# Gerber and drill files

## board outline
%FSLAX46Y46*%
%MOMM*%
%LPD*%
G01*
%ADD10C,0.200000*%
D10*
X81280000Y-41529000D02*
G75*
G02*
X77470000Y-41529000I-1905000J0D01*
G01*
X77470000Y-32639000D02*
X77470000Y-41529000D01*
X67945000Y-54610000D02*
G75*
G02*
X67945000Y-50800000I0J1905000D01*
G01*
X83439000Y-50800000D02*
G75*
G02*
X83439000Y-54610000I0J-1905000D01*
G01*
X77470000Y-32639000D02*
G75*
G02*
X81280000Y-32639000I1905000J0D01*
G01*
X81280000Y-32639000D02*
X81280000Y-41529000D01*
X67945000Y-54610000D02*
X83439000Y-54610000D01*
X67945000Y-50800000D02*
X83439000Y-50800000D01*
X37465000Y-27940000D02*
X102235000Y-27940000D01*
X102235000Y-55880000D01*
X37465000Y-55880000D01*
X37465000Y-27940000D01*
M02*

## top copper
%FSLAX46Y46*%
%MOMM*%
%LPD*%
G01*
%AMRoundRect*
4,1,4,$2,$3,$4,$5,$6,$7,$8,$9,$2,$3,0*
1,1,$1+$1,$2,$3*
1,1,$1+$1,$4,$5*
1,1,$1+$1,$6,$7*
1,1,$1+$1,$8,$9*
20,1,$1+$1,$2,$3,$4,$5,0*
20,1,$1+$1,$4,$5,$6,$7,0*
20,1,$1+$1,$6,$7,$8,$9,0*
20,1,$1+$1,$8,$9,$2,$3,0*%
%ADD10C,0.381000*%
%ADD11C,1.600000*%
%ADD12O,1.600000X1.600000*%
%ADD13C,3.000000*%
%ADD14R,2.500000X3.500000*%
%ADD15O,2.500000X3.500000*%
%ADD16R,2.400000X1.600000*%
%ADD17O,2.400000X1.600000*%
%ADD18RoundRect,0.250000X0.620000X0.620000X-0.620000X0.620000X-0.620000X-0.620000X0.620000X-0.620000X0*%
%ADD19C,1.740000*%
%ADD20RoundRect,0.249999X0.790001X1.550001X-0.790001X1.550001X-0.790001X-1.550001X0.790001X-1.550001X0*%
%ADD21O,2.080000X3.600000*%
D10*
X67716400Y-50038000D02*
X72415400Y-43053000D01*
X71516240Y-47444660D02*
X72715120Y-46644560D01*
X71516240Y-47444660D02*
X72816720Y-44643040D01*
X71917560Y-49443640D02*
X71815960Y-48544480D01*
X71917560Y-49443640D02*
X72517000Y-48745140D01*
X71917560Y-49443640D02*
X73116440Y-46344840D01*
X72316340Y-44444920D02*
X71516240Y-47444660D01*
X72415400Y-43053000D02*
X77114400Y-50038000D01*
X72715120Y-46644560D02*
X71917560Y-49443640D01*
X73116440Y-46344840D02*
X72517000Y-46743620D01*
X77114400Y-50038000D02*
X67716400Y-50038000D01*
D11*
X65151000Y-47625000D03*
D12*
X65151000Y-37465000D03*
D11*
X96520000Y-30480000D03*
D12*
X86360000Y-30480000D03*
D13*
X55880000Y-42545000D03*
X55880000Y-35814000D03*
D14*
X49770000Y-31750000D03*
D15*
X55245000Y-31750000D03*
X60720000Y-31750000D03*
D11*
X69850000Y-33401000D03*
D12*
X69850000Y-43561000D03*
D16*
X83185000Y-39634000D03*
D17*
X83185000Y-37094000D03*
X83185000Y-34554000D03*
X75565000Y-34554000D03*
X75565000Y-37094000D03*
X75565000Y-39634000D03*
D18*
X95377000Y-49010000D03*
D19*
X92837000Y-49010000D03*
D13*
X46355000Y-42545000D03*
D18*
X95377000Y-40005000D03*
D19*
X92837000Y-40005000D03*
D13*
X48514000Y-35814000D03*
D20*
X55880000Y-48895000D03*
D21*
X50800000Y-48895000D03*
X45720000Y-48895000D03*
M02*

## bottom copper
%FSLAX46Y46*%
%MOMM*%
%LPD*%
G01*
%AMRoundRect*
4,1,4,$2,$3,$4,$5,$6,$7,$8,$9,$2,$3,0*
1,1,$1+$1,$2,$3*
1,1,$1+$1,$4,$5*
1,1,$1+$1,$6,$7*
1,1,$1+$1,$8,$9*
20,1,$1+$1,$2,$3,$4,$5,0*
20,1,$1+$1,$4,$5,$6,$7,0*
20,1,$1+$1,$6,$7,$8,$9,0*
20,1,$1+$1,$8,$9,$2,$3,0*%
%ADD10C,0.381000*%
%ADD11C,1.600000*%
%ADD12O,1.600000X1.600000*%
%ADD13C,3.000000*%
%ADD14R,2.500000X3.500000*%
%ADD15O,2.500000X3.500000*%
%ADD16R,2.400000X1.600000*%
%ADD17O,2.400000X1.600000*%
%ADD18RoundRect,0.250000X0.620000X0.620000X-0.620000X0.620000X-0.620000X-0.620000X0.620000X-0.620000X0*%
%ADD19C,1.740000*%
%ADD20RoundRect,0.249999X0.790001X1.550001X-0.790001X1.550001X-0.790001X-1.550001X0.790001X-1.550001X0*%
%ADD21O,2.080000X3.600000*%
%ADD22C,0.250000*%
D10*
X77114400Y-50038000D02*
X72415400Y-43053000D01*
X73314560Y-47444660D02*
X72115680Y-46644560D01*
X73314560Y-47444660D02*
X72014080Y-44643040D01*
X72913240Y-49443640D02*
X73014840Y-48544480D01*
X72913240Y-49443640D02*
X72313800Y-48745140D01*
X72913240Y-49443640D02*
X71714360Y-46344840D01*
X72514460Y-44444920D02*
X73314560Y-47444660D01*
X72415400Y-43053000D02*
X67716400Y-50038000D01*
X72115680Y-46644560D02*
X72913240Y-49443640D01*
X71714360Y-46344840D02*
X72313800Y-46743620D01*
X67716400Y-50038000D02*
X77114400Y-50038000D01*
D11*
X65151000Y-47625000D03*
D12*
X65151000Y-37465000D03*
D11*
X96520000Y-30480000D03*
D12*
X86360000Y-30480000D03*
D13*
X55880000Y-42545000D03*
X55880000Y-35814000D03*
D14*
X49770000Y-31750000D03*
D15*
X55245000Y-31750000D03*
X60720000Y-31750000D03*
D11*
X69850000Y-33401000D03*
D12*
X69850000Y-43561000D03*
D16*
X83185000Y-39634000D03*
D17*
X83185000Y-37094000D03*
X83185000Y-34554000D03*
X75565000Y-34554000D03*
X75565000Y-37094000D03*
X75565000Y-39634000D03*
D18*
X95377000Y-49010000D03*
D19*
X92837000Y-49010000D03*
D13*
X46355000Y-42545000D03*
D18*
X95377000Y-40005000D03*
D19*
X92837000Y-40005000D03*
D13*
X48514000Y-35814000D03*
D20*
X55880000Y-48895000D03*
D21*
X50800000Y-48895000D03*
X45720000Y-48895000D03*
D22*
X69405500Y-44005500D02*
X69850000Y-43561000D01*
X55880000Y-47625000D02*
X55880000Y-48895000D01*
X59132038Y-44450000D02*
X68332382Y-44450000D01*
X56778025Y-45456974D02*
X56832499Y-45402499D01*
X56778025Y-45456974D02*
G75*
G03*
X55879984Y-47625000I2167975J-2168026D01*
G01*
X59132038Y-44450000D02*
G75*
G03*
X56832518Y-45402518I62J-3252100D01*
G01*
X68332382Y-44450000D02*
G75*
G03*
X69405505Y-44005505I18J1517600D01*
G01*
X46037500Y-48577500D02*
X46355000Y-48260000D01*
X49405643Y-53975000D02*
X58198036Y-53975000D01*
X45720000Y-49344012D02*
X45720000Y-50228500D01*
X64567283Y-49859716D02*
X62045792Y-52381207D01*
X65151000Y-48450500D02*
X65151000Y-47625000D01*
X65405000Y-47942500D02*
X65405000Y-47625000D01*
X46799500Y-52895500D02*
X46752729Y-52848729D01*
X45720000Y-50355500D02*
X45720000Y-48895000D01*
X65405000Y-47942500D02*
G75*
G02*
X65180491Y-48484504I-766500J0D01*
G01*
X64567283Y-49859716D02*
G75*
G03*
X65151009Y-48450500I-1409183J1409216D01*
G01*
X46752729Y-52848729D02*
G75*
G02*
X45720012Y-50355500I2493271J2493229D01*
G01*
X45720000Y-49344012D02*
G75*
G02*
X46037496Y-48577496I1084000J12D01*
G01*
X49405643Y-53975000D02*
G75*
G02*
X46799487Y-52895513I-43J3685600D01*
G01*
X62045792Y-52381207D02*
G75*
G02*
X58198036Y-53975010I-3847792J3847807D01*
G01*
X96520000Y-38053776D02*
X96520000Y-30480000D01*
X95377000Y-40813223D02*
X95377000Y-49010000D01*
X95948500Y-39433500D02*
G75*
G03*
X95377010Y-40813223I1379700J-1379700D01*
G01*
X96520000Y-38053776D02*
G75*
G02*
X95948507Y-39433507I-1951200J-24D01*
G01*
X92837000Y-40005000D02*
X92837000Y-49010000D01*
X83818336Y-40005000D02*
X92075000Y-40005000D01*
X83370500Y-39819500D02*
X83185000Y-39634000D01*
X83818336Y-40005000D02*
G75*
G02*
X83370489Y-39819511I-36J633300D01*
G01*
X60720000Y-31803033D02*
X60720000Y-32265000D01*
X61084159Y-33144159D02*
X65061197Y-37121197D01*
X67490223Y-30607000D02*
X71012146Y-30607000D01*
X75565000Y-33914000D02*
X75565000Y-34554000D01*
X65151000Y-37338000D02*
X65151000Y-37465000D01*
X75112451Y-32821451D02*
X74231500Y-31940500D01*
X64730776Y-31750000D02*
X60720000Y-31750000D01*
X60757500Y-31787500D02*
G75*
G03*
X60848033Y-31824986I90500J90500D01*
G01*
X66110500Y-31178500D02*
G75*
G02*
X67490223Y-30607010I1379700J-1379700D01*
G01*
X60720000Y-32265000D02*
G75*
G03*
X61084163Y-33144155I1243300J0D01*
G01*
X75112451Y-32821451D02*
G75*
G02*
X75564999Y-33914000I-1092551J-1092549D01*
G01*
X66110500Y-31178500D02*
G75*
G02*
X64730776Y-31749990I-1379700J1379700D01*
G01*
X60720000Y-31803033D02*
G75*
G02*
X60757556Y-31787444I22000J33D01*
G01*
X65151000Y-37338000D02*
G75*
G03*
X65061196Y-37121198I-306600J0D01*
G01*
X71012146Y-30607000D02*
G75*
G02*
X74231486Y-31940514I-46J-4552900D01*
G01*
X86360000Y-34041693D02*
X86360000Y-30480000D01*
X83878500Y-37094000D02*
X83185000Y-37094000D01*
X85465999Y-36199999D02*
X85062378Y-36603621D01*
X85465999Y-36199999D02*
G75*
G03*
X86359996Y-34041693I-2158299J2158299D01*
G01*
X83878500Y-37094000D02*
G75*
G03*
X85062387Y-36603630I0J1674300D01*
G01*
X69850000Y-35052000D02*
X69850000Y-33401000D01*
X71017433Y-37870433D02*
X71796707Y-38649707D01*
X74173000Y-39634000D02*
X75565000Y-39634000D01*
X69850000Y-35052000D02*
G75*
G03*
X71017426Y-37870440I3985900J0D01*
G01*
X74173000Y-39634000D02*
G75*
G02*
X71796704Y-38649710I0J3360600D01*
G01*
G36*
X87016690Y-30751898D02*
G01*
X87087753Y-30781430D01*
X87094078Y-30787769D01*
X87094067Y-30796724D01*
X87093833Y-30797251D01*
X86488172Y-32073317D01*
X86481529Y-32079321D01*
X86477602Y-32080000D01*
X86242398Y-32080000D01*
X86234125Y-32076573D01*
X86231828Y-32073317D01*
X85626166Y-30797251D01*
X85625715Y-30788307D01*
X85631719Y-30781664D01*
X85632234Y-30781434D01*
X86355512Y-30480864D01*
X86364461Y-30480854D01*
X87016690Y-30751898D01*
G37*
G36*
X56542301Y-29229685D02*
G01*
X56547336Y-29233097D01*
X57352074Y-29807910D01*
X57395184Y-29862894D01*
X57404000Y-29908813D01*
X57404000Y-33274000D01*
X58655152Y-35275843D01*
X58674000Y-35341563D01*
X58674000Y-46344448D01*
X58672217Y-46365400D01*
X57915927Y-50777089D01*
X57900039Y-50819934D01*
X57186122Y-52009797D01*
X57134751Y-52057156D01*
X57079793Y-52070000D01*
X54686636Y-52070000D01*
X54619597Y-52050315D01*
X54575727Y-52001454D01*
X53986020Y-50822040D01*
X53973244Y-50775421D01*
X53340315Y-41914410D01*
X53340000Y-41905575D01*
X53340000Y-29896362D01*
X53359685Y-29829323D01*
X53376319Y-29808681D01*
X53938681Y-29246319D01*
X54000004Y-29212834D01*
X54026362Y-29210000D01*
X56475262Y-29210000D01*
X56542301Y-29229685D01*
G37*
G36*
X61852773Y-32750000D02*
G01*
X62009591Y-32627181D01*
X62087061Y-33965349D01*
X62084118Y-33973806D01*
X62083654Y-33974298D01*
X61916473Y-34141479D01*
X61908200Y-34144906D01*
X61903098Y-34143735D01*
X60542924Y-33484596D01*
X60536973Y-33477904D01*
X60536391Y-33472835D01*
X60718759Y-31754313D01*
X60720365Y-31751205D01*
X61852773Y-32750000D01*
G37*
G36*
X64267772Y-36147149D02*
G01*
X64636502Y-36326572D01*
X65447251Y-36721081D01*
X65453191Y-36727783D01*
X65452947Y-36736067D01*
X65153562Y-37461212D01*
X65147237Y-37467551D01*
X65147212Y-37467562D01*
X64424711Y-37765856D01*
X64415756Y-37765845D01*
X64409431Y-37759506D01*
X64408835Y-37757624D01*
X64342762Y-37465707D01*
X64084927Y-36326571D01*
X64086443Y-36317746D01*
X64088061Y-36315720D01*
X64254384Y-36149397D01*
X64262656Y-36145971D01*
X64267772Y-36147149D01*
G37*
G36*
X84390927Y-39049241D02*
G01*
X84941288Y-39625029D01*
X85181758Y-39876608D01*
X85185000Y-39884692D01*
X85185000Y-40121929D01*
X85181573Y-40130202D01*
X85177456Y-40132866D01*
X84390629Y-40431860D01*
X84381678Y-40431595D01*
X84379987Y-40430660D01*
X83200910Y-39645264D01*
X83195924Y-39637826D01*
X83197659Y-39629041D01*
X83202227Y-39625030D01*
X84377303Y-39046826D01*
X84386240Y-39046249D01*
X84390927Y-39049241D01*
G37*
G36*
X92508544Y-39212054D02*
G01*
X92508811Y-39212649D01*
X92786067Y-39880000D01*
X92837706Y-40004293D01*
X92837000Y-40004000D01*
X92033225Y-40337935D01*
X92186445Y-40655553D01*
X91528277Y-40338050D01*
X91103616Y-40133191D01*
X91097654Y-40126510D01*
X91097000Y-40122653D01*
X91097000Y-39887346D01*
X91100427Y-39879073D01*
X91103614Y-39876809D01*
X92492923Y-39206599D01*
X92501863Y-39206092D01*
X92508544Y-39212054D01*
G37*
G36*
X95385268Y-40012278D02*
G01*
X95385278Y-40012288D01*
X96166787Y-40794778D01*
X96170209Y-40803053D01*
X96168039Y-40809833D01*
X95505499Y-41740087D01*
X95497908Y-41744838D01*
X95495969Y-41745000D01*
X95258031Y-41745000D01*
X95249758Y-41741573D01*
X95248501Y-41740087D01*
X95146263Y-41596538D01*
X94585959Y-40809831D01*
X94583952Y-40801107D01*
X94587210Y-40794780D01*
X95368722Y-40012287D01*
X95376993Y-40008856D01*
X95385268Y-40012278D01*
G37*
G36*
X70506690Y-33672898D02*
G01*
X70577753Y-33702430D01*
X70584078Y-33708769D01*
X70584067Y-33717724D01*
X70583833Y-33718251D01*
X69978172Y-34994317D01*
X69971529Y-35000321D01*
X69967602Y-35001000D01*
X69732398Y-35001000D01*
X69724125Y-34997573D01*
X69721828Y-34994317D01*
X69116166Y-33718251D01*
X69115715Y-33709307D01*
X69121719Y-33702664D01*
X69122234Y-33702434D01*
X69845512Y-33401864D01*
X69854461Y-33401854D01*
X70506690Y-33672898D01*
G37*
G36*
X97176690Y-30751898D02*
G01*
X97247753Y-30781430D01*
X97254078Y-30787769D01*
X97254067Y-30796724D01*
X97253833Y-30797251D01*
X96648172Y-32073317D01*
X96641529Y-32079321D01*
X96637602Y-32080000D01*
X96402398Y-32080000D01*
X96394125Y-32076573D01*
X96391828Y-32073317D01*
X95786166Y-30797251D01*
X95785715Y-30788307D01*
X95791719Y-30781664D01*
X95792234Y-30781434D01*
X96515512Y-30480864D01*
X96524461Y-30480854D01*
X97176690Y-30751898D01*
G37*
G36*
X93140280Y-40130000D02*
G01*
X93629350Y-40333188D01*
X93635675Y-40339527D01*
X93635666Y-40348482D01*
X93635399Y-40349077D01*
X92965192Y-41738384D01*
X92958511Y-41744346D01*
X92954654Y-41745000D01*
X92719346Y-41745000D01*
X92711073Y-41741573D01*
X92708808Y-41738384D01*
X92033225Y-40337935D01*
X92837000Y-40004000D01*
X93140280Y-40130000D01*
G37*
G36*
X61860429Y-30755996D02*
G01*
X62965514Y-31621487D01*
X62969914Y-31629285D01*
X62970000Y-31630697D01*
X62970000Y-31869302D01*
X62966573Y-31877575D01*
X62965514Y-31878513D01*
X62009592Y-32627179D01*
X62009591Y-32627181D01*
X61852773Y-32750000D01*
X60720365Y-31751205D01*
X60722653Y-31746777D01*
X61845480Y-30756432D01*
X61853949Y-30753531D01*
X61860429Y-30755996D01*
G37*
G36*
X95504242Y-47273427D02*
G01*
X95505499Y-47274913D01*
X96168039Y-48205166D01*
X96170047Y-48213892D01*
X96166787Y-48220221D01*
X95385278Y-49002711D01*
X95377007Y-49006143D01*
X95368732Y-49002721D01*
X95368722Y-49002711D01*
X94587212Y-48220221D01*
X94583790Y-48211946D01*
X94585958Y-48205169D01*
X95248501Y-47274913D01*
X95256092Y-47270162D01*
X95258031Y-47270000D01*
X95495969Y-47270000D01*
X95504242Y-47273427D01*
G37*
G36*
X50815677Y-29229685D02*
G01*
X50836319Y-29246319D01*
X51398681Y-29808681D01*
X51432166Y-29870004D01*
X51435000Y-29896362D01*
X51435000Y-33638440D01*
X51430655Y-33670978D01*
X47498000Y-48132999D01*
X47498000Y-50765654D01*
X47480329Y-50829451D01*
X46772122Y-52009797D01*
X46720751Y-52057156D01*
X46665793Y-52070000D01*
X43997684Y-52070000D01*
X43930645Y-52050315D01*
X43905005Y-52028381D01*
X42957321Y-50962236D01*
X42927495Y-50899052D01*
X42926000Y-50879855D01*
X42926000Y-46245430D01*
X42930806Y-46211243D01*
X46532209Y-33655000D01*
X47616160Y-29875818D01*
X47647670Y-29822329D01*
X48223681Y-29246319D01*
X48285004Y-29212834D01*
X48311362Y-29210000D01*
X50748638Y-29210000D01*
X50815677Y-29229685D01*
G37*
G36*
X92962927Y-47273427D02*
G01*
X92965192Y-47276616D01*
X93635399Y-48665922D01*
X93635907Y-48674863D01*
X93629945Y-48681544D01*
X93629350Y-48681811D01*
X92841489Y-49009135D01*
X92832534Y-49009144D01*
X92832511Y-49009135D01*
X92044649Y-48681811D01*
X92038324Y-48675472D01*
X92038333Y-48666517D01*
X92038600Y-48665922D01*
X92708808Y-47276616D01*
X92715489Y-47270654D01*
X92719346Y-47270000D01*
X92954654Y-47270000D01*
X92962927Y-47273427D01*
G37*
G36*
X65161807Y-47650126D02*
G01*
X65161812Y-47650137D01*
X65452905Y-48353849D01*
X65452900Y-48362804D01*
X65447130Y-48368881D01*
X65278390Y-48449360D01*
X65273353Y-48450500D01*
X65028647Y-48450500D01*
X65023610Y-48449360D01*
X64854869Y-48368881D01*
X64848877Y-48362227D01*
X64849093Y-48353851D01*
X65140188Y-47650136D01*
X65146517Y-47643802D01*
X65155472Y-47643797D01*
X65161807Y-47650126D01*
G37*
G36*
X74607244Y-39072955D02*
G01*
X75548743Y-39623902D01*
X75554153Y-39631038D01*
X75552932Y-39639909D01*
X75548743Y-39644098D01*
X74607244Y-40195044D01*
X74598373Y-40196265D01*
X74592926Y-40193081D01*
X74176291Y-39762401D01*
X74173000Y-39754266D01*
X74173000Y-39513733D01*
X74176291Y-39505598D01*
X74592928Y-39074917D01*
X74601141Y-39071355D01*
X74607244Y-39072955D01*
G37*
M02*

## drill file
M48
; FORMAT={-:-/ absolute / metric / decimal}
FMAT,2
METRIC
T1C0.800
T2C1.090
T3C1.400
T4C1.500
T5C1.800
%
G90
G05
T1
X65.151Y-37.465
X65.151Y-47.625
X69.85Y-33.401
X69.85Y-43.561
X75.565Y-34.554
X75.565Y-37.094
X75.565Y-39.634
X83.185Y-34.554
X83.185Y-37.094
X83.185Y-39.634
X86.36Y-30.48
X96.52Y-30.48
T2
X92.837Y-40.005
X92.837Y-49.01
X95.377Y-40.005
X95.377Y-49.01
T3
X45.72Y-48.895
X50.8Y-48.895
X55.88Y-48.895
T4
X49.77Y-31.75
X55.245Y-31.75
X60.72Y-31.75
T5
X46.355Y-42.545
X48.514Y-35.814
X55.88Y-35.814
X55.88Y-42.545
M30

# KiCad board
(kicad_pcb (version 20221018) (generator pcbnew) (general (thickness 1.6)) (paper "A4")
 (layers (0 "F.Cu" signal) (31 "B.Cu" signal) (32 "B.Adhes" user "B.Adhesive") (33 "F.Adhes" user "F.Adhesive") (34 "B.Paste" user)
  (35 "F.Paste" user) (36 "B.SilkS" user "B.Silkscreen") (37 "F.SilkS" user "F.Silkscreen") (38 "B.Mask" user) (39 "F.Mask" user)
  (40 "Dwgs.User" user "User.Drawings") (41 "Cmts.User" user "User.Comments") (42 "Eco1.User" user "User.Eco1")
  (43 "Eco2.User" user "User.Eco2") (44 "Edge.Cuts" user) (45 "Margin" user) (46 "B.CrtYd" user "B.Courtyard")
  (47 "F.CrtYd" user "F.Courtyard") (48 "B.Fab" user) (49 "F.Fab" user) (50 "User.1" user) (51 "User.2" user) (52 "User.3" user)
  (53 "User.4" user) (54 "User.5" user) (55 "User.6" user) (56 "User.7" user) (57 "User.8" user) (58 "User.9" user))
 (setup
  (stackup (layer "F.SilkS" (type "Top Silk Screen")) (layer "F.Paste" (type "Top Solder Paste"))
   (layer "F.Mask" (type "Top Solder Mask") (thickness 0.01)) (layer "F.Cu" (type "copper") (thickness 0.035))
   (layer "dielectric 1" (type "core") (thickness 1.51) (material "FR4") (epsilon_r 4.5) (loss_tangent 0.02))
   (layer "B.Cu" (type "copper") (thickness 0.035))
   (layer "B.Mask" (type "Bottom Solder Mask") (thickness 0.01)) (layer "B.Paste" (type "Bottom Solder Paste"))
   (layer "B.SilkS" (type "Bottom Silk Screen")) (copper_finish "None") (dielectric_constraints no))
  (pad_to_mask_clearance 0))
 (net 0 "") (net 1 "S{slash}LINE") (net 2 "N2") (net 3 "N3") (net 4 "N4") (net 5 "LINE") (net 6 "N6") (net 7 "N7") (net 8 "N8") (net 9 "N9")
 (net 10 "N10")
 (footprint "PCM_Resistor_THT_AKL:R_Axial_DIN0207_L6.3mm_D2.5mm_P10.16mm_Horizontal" (layer "F.Cu") (at 65.151 47.625 90)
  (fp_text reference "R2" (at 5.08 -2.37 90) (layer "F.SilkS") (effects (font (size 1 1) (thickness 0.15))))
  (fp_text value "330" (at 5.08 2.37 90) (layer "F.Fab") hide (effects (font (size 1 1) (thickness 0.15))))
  (pad "1" thru_hole circle (at 0 0 90) (size 1.6 1.6) (drill 0.8) (layers "*.Cu" "*.Mask") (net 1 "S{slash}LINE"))
  (pad "2" thru_hole oval (at 10.16 0 90) (size 1.6 1.6) (drill 0.8) (layers "*.Cu" "*.Mask") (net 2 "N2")))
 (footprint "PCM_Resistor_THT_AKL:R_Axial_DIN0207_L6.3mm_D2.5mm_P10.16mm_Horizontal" (layer "F.Cu") (at 96.52 30.48 180)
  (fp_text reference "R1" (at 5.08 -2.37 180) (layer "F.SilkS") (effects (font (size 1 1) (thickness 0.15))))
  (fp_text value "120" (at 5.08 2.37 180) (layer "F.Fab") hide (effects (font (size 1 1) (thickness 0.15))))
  (pad "1" thru_hole circle (at 0 0 180) (size 1.6 1.6) (drill 0.8) (layers "*.Cu" "*.Mask") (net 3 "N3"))
  (pad "2" thru_hole oval (at 10.16 0 180) (size 1.6 1.6) (drill 0.8) (layers "*.Cu" "*.Mask") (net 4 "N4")))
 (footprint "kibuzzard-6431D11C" (layer "F.Cu") (at 39.624 41.91 90)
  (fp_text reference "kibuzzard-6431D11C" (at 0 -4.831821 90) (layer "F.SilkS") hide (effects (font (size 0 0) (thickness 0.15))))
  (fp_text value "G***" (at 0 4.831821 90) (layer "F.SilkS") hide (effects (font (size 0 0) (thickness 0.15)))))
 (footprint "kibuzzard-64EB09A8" (layer "F.Cu") (at 100.8126 41.91 -90)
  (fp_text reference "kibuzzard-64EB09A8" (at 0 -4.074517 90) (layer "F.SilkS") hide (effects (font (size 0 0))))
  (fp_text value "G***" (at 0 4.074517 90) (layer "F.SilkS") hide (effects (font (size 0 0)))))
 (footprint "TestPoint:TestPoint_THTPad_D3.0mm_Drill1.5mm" (layer "F.Cu") (at 55.88 42.545)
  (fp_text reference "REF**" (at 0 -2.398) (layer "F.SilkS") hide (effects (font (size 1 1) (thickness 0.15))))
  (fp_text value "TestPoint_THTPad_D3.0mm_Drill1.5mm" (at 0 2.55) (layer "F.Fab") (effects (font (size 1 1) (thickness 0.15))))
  (pad "1" thru_hole circle (at 0 0) (size 3 3) (drill 1.8) (layers "*.Cu" "*.Mask") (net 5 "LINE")))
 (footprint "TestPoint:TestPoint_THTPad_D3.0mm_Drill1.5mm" (layer "F.Cu") (at 55.88 35.814)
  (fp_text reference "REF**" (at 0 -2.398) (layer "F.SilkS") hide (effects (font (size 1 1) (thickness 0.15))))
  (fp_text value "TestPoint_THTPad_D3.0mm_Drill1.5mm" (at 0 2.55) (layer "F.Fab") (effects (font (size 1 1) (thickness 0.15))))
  (pad "1" thru_hole circle (at 0 0) (size 3 3) (drill 1.8) (layers "*.Cu" "*.Mask") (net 5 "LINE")))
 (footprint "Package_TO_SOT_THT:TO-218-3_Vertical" (layer "F.Cu") (at 49.77 31.75)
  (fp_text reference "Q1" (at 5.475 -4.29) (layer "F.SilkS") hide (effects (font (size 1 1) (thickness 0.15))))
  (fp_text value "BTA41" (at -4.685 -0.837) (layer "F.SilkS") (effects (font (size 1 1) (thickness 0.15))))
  (pad "1" thru_hole rect (at 0 0) (size 2.5 3.5) (drill 1.5) (layers "*.Cu" "*.Mask") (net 1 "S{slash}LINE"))
  (pad "2" thru_hole oval (at 5.475 0) (size 2.5 3.5) (drill 1.5) (layers "*.Cu" "*.Mask") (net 5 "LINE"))
  (pad "3" thru_hole oval (at 10.95 0) (size 2.5 3.5) (drill 1.5) (layers "*.Cu" "*.Mask") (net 2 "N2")))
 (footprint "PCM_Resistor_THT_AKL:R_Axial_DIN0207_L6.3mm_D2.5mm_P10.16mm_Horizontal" (layer "F.Cu") (at 69.85 33.401 -90)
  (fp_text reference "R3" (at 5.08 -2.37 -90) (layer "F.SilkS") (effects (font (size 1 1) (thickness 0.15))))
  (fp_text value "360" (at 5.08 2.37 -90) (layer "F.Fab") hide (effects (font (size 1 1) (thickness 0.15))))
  (pad "1" thru_hole circle (at 0 0 270) (size 1.6 1.6) (drill 0.8) (layers "*.Cu" "*.Mask") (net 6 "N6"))
  (pad "2" thru_hole oval (at 10.16 0 270) (size 1.6 1.6) (drill 0.8) (layers "*.Cu" "*.Mask") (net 5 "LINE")))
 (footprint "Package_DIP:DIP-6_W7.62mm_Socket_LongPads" (layer "F.Cu") (at 83.185 39.634 180)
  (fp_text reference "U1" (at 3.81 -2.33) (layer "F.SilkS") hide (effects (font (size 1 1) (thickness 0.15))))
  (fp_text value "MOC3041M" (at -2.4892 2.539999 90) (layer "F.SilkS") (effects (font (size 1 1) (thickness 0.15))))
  (pad "1" thru_hole rect (at 0 0 180) (size 2.4 1.6) (drill 0.8) (layers "*.Cu" "*.Mask") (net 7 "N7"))
  (pad "2" thru_hole oval (at 0 2.54 180) (size 2.4 1.6) (drill 0.8) (layers "*.Cu" "*.Mask") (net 4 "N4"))
  (pad "3" thru_hole oval (at 0 5.08 180) (size 2.4 1.6) (drill 0.8) (layers "*.Cu" "*.Mask") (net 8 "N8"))
  (pad "4" thru_hole oval (at 7.62 5.08 180) (size 2.4 1.6) (drill 0.8) (layers "*.Cu" "*.Mask") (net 2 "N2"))
  (pad "5" thru_hole oval (at 7.62 2.54 180) (size 2.4 1.6) (drill 0.8) (layers "*.Cu" "*.Mask") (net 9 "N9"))
  (pad "6" thru_hole oval (at 7.62 0 180) (size 2.4 1.6) (drill 0.8) (layers "*.Cu" "*.Mask") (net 6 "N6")))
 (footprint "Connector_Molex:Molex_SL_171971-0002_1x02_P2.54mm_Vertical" (layer "F.Cu") (at 95.377 49.01 180)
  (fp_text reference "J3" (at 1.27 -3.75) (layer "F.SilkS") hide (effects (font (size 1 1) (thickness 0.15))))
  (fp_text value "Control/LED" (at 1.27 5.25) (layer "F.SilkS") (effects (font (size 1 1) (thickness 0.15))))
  (pad "1" thru_hole roundrect (at 0 0 180) (size 1.74 1.74) (drill 1.09) (layers "*.Cu" "*.Mask") (roundrect_rratio 0.143678) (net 3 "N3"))
  (pad "2" thru_hole circle (at 2.54 0 180) (size 1.74 1.74) (drill 1.09) (layers "*.Cu" "*.Mask") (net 7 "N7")))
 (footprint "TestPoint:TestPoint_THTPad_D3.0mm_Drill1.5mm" (layer "F.Cu") (at 46.355 42.545)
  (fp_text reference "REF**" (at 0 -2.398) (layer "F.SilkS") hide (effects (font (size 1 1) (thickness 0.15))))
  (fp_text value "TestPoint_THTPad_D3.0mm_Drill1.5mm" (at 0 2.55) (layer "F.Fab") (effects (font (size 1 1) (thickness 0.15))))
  (pad "1" thru_hole circle (at 0 0) (size 3 3) (drill 1.8) (layers "*.Cu" "*.Mask") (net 1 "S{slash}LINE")))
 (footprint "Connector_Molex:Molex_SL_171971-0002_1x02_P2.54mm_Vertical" (layer "F.Cu") (at 95.377 40.005 180)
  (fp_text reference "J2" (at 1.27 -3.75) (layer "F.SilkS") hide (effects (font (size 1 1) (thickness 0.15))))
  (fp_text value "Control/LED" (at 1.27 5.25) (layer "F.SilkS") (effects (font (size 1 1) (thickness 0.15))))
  (pad "1" thru_hole roundrect (at 0 0 180) (size 1.74 1.74) (drill 1.09) (layers "*.Cu" "*.Mask") (roundrect_rratio 0.143678) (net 3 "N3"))
  (pad "2" thru_hole circle (at 2.54 0 180) (size 1.74 1.74) (drill 1.09) (layers "*.Cu" "*.Mask") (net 7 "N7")))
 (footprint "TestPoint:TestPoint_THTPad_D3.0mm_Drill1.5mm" (layer "F.Cu") (at 48.514 35.814)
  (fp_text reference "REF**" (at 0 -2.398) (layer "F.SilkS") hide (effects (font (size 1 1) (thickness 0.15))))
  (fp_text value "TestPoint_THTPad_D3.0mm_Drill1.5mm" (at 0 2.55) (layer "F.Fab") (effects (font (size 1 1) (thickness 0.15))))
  (pad "1" thru_hole circle (at 0 0) (size 3 3) (drill 1.8) (layers "*.Cu" "*.Mask") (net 1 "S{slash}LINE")))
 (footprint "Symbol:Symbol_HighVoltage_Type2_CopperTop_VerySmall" (layer "F.Cu") (at 72.4154 47.244)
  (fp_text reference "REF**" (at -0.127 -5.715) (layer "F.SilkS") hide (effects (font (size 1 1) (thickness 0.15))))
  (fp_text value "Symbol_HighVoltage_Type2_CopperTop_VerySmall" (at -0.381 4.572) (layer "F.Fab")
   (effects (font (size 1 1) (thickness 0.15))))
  (fp_line (start -4.699 2.794) (end 0 -4.191) (stroke (width 0.381) (type solid)) (layer "F.Cu"))
  (fp_line (start -0.89916 0.20066) (end 0.29972 -0.59944) (stroke (width 0.381) (type solid)) (layer "F.Cu"))
  (fp_line (start -0.89916 0.20066) (end 0.40132 -2.60096) (stroke (width 0.381) (type solid)) (layer "F.Cu"))
  (fp_line (start -0.49784 2.19964) (end -0.59944 1.30048) (stroke (width 0.381) (type solid)) (layer "F.Cu"))
  (fp_line (start -0.49784 2.19964) (end 0.1016 1.50114) (stroke (width 0.381) (type solid)) (layer "F.Cu"))
  (fp_line (start -0.49784 2.19964) (end 0.70104 -0.89916) (stroke (width 0.381) (type solid)) (layer "F.Cu"))
  (fp_line (start -0.09906 -2.79908) (end -0.89916 0.20066) (stroke (width 0.381) (type solid)) (layer "F.Cu"))
  (fp_line (start 0 -4.191) (end 4.699 2.794) (stroke (width 0.381) (type solid)) (layer "F.Cu"))
  (fp_line (start 0.29972 -0.59944) (end -0.49784 2.19964) (stroke (width 0.381) (type solid)) (layer "F.Cu"))
  (fp_line (start 0.70104 -0.89916) (end 0.1016 -0.50038) (stroke (width 0.381) (type solid)) (layer "F.Cu"))
  (fp_line (start 4.699 2.794) (end -4.699 2.794) (stroke (width 0.381) (type solid)) (layer "F.Cu")))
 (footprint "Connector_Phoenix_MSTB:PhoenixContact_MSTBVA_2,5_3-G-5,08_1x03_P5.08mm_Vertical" (layer "F.Cu") (at 55.88 48.895 180)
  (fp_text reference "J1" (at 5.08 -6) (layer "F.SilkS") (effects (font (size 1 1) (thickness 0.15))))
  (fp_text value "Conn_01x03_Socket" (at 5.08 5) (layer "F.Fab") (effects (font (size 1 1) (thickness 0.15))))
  (pad "1" thru_hole roundrect (at 0 0 180) (size 2.08 3.6) (drill 1.4) (layers "*.Cu" "*.Mask") (roundrect_rratio 0.120192) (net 5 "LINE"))
  (pad "2" thru_hole oval (at 5.08 0 180) (size 2.08 3.6) (drill 1.4) (layers "*.Cu" "*.Mask") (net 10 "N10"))
  (pad "3" thru_hole oval (at 10.16 0 180) (size 2.08 3.6) (drill 1.4) (layers "*.Cu" "*.Mask") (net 1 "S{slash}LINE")))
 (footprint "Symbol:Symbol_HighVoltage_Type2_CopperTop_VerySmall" (layer "B.Cu") (at 72.4154 47.244 180)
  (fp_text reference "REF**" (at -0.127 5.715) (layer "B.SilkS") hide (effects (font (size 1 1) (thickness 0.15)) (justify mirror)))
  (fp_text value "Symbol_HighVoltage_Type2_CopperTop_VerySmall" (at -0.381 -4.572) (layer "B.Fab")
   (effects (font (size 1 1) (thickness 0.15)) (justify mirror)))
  (fp_line (start -4.699 -2.794) (end 0 4.191) (stroke (width 0.381) (type solid)) (layer "B.Cu"))
  (fp_line (start -0.89916 -0.20066) (end 0.29972 0.59944) (stroke (width 0.381) (type solid)) (layer "B.Cu"))
  (fp_line (start -0.89916 -0.20066) (end 0.40132 2.60096) (stroke (width 0.381) (type solid)) (layer "B.Cu"))
  (fp_line (start -0.49784 -2.19964) (end -0.59944 -1.30048) (stroke (width 0.381) (type solid)) (layer "B.Cu"))
  (fp_line (start -0.49784 -2.19964) (end 0.1016 -1.50114) (stroke (width 0.381) (type solid)) (layer "B.Cu"))
  (fp_line (start -0.49784 -2.19964) (end 0.70104 0.89916) (stroke (width 0.381) (type solid)) (layer "B.Cu"))
  (fp_line (start -0.09906 2.79908) (end -0.89916 -0.20066) (stroke (width 0.381) (type solid)) (layer "B.Cu"))
  (fp_line (start 0 4.191) (end 4.699 -2.794) (stroke (width 0.381) (type solid)) (layer "B.Cu"))
  (fp_line (start 0.29972 0.59944) (end -0.49784 -2.19964) (stroke (width 0.381) (type solid)) (layer "B.Cu"))
  (fp_line (start 0.70104 0.89916) (end 0.1016 0.50038) (stroke (width 0.381) (type solid)) (layer "B.Cu"))
  (fp_line (start 4.699 -2.794) (end -4.699 -2.794) (stroke (width 0.381) (type solid)) (layer "B.Cu")))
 (gr_arc (start 81.28 41.529) (mid 79.375 43.434) (end 77.47 41.529) (stroke (width 0.2) (type default)) (layer "Edge.Cuts"))
 (gr_line (start 77.47 32.639) (end 77.47 41.529) (stroke (width 0.2) (type default)) (layer "Edge.Cuts"))
 (gr_arc (start 67.945 54.61) (mid 66.04 52.705) (end 67.945 50.8) (stroke (width 0.2) (type default)) (layer "Edge.Cuts"))
 (gr_arc (start 83.439 50.8) (mid 85.344 52.705) (end 83.439 54.61) (stroke (width 0.2) (type default)) (layer "Edge.Cuts"))
 (gr_arc (start 77.47 32.639) (mid 79.375 30.734) (end 81.28 32.639) (stroke (width 0.2) (type default)) (layer "Edge.Cuts"))
 (gr_line (start 81.28 32.639) (end 81.28 41.529) (stroke (width 0.2) (type default)) (layer "Edge.Cuts"))
 (gr_line (start 67.945 54.61) (end 83.439 54.61) (stroke (width 0.2) (type default)) (layer "Edge.Cuts"))
 (gr_line (start 67.945 50.8) (end 83.439 50.8) (stroke (width 0.2) (type default)) (layer "Edge.Cuts"))
 (gr_rect (start 37.465 27.94) (end 102.235 55.88) (stroke (width 0.2) (type default)) (fill none) (layer "Edge.Cuts"))
 (segment (start 69.4055 44.0055) (end 69.85 43.561) (width 0.25) (layer "B.Cu") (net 5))
 (segment (start 55.88 47.625) (end 55.88 48.895) (width 0.25) (layer "B.Cu") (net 5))
 (segment (start 59.132038 44.45) (end 68.332382 44.45) (width 0.25) (layer "B.Cu") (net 5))
 (segment (start 56.778025 45.456974) (end 56.832499 45.402499) (width 0.25) (layer "B.Cu") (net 5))
 (arc (start 56.778025 45.456974) (mid 56.113389 46.451672) (end 55.88 47.625) (width 0.25) (layer "B.Cu") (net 5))
 (arc (start 59.132038 44.45) (mid 57.887537 44.69755) (end 56.832499 45.402499) (width 0.25) (layer "B.Cu") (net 5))
 (arc (start 68.332382 44.45) (mid 68.913149 44.334478) (end 69.4055 44.0055) (width 0.25) (layer "B.Cu") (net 5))
 (segment (start 46.0375 48.5775) (end 46.355 48.26) (width 0.25) (layer "B.Cu") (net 1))
 (segment (start 49.405643 53.975) (end 58.198036 53.975) (width 0.25) (layer "B.Cu") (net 1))
 (segment (start 45.72 49.344012) (end 45.72 50.2285) (width 0.25) (layer "B.Cu") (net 1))
 (segment (start 64.567283 49.859716) (end 62.045792 52.381207) (width 0.25) (layer "B.Cu") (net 1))
 (segment (start 65.151 48.4505) (end 65.151 47.625) (width 0.25) (layer "B.Cu") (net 1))
 (segment (start 65.405 47.9425) (end 65.405 47.625) (width 0.25) (layer "B.Cu") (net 1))
 (segment (start 46.7995 52.8955) (end 46.752729 52.848729) (width 0.25) (layer "B.Cu") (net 1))
 (segment (start 45.72 50.3555) (end 45.72 48.895) (width 0.25) (layer "B.Cu") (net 1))
 (arc (start 65.405 47.9425) (mid 65.346652 48.235831) (end 65.180493 48.484506) (width 0.25) (layer "B.Cu") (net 1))
 (arc (start 64.567283 49.859716) (mid 64.999296 49.213162) (end 65.151 48.4505) (width 0.25) (layer "B.Cu") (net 1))
 (arc (start 46.752729 52.848729) (mid 45.988397 51.704825) (end 45.72 50.3555) (width 0.25) (layer "B.Cu") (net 1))
 (arc (start 45.72 49.344012) (mid 45.802515 48.929178) (end 46.0375 48.5775) (width 0.25) (layer "B.Cu") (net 1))
 (arc (start 49.405643 53.975) (mid 47.995208 53.694447) (end 46.7995 52.8955) (width 0.25) (layer "B.Cu") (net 1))
 (arc (start 62.045792 52.381207) (mid 60.280426 53.560786) (end 58.198036 53.975) (width 0.25) (layer "B.Cu") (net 1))
 (segment (start 96.52 38.053776) (end 96.52 30.48) (width 0.25) (layer "B.Cu") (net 3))
 (segment (start 95.377 40.813223) (end 95.377 49.01) (width 0.25) (layer "B.Cu") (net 3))
 (arc (start 95.9485 39.4335) (mid 95.525528 40.066522) (end 95.377 40.813223) (width 0.25) (layer "B.Cu") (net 3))
 (arc (start 96.52 38.053776) (mid 96.371471 38.800477) (end 95.9485 39.4335) (width 0.25) (layer "B.Cu") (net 3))
 (segment (start 92.837 40.005) (end 92.837 49.01) (width 0.25) (layer "B.Cu") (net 7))
 (segment (start 83.818336 40.005) (end 92.075 40.005) (width 0.25) (layer "B.Cu") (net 7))
 (segment (start 83.3705 39.8195) (end 83.185 39.634) (width 0.25) (layer "B.Cu") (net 7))
 (arc (start 83.818336 40.005) (mid 83.575969 39.95679) (end 83.3705 39.8195) (width 0.25) (layer "B.Cu") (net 7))
 (segment (start 60.72 31.803033) (end 60.72 32.265) (width 0.25) (layer "B.Cu") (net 2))
 (segment (start 61.084159 33.144159) (end 65.061197 37.121197) (width 0.25) (layer "B.Cu") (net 2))
 (segment (start 67.490223 30.607) (end 71.012146 30.607) (width 0.25) (layer "B.Cu") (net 2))
 (segment (start 75.565 33.914) (end 75.565 34.554) (width 0.25) (layer "B.Cu") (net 2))
 (segment (start 65.151 37.338) (end 65.151 37.465) (width 0.25) (layer "B.Cu") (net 2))
 (segment (start 75.112451 32.821451) (end 74.2315 31.9405) (width 0.25) (layer "B.Cu") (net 2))
 (segment (start 64.730776 31.75) (end 60.72 31.75) (width 0.25) (layer "B.Cu") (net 2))
 (arc (start 60.7575 31.7875) (mid 60.799036 31.815254) (end 60.848033 31.825) (width 0.25) (layer "B.Cu") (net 2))
 (arc (start 66.1105 31.1785) (mid 66.743522 30.755528) (end 67.490223 30.607) (width 0.25) (layer "B.Cu") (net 2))
 (arc (start 60.72 32.265) (mid 60.814643 32.740796) (end 61.084159 33.144159) (width 0.25) (layer "B.Cu") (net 2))
 (arc (start 75.112451 32.821451) (mid 75.447386 33.322716) (end 75.565 33.914) (width 0.25) (layer "B.Cu") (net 2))
 (arc (start 66.1105 31.1785) (mid 65.477477 31.601471) (end 64.730776 31.75) (width 0.25) (layer "B.Cu") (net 2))
 (arc (start 60.72 31.803033) (mid 60.73356 31.782738) (end 60.7575 31.7875) (width 0.25) (layer "B.Cu") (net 2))
 (arc (start 65.151 37.338) (mid 65.12766 37.220667) (end 65.061197 37.121197) (width 0.25) (layer "B.Cu") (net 2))
 (arc (start 71.012146 30.607) (mid 72.754447 30.953565) (end 74.2315 31.9405) (width 0.25) (layer "B.Cu") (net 2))
 (segment (start 86.36 34.041693) (end 86.36 30.48) (width 0.25) (layer "B.Cu") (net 4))
 (segment (start 83.8785 37.094) (end 83.185 37.094) (width 0.25) (layer "B.Cu") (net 4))
 (segment (start 85.465999 36.199999) (end 85.062378 36.603621) (width 0.25) (layer "B.Cu") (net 4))
 (arc (start 85.465999 36.199999) (mid 86.127656 35.20976) (end 86.36 34.041693) (width 0.25) (layer "B.Cu") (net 4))
 (arc (start 83.8785 37.094) (mid 84.51921 36.966554) (end 85.062378 36.603621) (width 0.25) (layer "B.Cu") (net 4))
 (segment (start 69.85 35.052) (end 69.85 33.401) (width 0.25) (layer "B.Cu") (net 6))
 (segment (start 71.017433 37.870433) (end 71.796707 38.649707) (width 0.25) (layer "B.Cu") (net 6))
 (segment (start 74.173 39.634) (end 75.565 39.634) (width 0.25) (layer "B.Cu") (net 6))
 (arc (start 69.85 35.052) (mid 70.153405 36.577325) (end 71.017433 37.870433) (width 0.25) (layer "B.Cu") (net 6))
 (arc (start 74.173 39.634) (mid 72.886959 39.37819) (end 71.796707 38.649707) (width 0.25) (layer "B.Cu") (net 6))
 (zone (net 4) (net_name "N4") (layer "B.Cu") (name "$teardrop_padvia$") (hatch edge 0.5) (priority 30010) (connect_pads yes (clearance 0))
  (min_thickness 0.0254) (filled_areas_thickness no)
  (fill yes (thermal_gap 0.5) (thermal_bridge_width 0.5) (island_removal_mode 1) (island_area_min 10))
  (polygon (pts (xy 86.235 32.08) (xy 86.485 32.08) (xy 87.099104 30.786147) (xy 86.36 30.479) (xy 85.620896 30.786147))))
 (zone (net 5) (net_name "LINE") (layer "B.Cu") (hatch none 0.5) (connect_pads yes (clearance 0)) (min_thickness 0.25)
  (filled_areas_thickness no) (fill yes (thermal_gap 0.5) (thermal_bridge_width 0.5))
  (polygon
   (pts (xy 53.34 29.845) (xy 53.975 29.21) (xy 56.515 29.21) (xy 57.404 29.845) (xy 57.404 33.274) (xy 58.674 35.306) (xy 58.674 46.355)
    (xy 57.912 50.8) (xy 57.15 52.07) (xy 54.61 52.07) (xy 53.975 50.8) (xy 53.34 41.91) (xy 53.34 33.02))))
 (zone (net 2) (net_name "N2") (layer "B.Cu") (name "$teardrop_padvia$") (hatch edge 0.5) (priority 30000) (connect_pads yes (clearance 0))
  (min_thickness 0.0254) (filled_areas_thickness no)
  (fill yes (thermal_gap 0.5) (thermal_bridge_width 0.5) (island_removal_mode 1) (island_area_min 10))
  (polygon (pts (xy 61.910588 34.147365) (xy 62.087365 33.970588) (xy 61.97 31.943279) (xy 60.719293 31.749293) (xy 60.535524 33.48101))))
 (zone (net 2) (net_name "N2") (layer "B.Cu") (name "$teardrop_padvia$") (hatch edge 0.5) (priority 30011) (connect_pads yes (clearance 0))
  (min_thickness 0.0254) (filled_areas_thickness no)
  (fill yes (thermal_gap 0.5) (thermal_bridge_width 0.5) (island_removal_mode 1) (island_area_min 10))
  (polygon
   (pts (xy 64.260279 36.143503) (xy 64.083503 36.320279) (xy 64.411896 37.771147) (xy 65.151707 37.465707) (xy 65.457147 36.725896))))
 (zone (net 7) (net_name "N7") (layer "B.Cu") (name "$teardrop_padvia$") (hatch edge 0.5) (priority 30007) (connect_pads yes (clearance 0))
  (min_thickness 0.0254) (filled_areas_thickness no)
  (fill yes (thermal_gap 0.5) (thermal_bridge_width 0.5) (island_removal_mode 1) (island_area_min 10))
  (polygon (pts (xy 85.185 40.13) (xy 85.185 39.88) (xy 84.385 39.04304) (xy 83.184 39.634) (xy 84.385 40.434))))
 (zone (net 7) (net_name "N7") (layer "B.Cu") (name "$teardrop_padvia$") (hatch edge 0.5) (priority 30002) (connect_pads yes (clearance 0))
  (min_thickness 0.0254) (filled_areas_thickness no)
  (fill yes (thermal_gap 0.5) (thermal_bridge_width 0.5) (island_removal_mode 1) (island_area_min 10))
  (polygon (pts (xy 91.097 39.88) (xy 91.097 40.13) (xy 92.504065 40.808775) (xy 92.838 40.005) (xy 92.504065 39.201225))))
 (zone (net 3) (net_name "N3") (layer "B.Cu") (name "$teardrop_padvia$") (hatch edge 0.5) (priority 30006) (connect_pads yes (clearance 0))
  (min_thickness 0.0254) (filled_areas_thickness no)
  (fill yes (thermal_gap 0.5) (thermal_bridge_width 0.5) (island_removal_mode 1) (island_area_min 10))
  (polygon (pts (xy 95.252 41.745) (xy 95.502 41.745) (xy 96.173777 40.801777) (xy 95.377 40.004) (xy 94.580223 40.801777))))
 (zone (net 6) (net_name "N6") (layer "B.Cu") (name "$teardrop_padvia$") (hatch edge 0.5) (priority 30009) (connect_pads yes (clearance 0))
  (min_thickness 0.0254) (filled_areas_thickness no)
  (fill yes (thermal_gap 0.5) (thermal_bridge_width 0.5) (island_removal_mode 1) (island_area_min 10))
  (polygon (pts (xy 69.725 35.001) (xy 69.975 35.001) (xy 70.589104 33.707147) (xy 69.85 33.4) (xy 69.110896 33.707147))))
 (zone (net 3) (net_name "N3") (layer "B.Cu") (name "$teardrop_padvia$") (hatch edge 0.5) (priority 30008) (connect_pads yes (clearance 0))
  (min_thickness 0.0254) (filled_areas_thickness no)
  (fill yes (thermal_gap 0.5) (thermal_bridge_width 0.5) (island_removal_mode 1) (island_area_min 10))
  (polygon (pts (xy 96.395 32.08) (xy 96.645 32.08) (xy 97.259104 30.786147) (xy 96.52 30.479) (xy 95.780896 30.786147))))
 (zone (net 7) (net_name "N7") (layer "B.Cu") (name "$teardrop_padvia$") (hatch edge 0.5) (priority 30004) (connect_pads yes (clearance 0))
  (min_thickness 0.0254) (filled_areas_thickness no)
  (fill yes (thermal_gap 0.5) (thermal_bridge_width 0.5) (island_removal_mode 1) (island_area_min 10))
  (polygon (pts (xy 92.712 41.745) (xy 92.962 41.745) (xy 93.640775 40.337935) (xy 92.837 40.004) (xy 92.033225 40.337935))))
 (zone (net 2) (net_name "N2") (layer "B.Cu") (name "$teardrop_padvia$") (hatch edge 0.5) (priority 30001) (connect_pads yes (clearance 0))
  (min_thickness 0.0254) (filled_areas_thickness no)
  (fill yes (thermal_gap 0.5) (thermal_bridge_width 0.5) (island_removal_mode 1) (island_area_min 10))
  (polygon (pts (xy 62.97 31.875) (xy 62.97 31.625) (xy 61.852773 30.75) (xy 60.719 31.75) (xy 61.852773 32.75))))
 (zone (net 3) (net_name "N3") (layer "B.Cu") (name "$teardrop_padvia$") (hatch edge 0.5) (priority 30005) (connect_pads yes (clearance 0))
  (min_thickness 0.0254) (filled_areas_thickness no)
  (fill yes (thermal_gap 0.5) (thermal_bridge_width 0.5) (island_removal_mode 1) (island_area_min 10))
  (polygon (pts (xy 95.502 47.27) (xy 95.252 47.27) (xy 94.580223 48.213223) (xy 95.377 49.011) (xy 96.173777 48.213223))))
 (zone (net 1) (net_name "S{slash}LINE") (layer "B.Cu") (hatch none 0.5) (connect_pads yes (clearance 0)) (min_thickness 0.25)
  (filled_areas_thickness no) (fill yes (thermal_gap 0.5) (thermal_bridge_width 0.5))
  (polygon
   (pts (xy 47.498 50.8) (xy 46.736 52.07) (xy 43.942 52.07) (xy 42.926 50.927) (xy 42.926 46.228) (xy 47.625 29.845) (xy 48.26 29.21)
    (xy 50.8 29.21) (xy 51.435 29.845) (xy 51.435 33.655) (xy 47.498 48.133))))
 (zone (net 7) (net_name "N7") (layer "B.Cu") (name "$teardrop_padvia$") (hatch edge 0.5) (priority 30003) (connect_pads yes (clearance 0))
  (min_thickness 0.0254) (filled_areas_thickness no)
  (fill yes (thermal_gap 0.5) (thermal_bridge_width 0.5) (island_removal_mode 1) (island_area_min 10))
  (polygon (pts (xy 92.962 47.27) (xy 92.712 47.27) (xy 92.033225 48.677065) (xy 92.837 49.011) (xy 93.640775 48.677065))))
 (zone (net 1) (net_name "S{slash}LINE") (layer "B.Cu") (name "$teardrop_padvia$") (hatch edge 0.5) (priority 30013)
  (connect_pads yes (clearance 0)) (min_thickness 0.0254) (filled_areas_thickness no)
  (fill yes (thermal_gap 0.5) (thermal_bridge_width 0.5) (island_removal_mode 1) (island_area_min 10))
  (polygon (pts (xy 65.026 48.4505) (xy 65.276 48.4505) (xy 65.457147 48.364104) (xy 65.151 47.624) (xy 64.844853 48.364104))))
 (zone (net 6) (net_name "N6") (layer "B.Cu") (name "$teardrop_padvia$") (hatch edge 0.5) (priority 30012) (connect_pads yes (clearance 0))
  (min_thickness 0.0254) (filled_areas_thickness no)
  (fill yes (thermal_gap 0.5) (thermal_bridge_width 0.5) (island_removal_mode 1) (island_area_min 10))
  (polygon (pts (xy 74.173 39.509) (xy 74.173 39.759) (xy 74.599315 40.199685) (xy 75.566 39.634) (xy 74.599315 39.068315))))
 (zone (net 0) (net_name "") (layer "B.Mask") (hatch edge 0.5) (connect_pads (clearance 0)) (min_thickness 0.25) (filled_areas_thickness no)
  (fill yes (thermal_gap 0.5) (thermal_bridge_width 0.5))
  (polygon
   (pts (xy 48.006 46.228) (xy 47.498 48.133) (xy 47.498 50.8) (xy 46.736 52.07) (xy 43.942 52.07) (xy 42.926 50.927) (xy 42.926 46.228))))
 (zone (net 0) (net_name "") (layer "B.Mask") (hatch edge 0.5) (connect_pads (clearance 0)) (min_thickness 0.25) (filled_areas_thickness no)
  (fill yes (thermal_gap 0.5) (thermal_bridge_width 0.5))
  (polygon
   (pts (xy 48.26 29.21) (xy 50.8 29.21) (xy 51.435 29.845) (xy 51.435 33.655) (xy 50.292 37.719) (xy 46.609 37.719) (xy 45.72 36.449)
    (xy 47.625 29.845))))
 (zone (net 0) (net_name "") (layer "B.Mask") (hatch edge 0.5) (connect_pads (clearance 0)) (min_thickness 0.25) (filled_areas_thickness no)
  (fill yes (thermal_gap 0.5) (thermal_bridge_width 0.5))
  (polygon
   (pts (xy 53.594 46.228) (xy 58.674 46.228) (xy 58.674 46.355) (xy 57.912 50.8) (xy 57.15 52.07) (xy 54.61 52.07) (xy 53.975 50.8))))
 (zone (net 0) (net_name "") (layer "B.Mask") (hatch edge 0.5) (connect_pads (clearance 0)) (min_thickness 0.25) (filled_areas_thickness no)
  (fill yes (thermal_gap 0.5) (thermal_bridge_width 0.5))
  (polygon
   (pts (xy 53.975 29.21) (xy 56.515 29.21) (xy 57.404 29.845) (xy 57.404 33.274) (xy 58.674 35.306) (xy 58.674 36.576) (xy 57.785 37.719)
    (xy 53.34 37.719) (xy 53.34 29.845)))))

